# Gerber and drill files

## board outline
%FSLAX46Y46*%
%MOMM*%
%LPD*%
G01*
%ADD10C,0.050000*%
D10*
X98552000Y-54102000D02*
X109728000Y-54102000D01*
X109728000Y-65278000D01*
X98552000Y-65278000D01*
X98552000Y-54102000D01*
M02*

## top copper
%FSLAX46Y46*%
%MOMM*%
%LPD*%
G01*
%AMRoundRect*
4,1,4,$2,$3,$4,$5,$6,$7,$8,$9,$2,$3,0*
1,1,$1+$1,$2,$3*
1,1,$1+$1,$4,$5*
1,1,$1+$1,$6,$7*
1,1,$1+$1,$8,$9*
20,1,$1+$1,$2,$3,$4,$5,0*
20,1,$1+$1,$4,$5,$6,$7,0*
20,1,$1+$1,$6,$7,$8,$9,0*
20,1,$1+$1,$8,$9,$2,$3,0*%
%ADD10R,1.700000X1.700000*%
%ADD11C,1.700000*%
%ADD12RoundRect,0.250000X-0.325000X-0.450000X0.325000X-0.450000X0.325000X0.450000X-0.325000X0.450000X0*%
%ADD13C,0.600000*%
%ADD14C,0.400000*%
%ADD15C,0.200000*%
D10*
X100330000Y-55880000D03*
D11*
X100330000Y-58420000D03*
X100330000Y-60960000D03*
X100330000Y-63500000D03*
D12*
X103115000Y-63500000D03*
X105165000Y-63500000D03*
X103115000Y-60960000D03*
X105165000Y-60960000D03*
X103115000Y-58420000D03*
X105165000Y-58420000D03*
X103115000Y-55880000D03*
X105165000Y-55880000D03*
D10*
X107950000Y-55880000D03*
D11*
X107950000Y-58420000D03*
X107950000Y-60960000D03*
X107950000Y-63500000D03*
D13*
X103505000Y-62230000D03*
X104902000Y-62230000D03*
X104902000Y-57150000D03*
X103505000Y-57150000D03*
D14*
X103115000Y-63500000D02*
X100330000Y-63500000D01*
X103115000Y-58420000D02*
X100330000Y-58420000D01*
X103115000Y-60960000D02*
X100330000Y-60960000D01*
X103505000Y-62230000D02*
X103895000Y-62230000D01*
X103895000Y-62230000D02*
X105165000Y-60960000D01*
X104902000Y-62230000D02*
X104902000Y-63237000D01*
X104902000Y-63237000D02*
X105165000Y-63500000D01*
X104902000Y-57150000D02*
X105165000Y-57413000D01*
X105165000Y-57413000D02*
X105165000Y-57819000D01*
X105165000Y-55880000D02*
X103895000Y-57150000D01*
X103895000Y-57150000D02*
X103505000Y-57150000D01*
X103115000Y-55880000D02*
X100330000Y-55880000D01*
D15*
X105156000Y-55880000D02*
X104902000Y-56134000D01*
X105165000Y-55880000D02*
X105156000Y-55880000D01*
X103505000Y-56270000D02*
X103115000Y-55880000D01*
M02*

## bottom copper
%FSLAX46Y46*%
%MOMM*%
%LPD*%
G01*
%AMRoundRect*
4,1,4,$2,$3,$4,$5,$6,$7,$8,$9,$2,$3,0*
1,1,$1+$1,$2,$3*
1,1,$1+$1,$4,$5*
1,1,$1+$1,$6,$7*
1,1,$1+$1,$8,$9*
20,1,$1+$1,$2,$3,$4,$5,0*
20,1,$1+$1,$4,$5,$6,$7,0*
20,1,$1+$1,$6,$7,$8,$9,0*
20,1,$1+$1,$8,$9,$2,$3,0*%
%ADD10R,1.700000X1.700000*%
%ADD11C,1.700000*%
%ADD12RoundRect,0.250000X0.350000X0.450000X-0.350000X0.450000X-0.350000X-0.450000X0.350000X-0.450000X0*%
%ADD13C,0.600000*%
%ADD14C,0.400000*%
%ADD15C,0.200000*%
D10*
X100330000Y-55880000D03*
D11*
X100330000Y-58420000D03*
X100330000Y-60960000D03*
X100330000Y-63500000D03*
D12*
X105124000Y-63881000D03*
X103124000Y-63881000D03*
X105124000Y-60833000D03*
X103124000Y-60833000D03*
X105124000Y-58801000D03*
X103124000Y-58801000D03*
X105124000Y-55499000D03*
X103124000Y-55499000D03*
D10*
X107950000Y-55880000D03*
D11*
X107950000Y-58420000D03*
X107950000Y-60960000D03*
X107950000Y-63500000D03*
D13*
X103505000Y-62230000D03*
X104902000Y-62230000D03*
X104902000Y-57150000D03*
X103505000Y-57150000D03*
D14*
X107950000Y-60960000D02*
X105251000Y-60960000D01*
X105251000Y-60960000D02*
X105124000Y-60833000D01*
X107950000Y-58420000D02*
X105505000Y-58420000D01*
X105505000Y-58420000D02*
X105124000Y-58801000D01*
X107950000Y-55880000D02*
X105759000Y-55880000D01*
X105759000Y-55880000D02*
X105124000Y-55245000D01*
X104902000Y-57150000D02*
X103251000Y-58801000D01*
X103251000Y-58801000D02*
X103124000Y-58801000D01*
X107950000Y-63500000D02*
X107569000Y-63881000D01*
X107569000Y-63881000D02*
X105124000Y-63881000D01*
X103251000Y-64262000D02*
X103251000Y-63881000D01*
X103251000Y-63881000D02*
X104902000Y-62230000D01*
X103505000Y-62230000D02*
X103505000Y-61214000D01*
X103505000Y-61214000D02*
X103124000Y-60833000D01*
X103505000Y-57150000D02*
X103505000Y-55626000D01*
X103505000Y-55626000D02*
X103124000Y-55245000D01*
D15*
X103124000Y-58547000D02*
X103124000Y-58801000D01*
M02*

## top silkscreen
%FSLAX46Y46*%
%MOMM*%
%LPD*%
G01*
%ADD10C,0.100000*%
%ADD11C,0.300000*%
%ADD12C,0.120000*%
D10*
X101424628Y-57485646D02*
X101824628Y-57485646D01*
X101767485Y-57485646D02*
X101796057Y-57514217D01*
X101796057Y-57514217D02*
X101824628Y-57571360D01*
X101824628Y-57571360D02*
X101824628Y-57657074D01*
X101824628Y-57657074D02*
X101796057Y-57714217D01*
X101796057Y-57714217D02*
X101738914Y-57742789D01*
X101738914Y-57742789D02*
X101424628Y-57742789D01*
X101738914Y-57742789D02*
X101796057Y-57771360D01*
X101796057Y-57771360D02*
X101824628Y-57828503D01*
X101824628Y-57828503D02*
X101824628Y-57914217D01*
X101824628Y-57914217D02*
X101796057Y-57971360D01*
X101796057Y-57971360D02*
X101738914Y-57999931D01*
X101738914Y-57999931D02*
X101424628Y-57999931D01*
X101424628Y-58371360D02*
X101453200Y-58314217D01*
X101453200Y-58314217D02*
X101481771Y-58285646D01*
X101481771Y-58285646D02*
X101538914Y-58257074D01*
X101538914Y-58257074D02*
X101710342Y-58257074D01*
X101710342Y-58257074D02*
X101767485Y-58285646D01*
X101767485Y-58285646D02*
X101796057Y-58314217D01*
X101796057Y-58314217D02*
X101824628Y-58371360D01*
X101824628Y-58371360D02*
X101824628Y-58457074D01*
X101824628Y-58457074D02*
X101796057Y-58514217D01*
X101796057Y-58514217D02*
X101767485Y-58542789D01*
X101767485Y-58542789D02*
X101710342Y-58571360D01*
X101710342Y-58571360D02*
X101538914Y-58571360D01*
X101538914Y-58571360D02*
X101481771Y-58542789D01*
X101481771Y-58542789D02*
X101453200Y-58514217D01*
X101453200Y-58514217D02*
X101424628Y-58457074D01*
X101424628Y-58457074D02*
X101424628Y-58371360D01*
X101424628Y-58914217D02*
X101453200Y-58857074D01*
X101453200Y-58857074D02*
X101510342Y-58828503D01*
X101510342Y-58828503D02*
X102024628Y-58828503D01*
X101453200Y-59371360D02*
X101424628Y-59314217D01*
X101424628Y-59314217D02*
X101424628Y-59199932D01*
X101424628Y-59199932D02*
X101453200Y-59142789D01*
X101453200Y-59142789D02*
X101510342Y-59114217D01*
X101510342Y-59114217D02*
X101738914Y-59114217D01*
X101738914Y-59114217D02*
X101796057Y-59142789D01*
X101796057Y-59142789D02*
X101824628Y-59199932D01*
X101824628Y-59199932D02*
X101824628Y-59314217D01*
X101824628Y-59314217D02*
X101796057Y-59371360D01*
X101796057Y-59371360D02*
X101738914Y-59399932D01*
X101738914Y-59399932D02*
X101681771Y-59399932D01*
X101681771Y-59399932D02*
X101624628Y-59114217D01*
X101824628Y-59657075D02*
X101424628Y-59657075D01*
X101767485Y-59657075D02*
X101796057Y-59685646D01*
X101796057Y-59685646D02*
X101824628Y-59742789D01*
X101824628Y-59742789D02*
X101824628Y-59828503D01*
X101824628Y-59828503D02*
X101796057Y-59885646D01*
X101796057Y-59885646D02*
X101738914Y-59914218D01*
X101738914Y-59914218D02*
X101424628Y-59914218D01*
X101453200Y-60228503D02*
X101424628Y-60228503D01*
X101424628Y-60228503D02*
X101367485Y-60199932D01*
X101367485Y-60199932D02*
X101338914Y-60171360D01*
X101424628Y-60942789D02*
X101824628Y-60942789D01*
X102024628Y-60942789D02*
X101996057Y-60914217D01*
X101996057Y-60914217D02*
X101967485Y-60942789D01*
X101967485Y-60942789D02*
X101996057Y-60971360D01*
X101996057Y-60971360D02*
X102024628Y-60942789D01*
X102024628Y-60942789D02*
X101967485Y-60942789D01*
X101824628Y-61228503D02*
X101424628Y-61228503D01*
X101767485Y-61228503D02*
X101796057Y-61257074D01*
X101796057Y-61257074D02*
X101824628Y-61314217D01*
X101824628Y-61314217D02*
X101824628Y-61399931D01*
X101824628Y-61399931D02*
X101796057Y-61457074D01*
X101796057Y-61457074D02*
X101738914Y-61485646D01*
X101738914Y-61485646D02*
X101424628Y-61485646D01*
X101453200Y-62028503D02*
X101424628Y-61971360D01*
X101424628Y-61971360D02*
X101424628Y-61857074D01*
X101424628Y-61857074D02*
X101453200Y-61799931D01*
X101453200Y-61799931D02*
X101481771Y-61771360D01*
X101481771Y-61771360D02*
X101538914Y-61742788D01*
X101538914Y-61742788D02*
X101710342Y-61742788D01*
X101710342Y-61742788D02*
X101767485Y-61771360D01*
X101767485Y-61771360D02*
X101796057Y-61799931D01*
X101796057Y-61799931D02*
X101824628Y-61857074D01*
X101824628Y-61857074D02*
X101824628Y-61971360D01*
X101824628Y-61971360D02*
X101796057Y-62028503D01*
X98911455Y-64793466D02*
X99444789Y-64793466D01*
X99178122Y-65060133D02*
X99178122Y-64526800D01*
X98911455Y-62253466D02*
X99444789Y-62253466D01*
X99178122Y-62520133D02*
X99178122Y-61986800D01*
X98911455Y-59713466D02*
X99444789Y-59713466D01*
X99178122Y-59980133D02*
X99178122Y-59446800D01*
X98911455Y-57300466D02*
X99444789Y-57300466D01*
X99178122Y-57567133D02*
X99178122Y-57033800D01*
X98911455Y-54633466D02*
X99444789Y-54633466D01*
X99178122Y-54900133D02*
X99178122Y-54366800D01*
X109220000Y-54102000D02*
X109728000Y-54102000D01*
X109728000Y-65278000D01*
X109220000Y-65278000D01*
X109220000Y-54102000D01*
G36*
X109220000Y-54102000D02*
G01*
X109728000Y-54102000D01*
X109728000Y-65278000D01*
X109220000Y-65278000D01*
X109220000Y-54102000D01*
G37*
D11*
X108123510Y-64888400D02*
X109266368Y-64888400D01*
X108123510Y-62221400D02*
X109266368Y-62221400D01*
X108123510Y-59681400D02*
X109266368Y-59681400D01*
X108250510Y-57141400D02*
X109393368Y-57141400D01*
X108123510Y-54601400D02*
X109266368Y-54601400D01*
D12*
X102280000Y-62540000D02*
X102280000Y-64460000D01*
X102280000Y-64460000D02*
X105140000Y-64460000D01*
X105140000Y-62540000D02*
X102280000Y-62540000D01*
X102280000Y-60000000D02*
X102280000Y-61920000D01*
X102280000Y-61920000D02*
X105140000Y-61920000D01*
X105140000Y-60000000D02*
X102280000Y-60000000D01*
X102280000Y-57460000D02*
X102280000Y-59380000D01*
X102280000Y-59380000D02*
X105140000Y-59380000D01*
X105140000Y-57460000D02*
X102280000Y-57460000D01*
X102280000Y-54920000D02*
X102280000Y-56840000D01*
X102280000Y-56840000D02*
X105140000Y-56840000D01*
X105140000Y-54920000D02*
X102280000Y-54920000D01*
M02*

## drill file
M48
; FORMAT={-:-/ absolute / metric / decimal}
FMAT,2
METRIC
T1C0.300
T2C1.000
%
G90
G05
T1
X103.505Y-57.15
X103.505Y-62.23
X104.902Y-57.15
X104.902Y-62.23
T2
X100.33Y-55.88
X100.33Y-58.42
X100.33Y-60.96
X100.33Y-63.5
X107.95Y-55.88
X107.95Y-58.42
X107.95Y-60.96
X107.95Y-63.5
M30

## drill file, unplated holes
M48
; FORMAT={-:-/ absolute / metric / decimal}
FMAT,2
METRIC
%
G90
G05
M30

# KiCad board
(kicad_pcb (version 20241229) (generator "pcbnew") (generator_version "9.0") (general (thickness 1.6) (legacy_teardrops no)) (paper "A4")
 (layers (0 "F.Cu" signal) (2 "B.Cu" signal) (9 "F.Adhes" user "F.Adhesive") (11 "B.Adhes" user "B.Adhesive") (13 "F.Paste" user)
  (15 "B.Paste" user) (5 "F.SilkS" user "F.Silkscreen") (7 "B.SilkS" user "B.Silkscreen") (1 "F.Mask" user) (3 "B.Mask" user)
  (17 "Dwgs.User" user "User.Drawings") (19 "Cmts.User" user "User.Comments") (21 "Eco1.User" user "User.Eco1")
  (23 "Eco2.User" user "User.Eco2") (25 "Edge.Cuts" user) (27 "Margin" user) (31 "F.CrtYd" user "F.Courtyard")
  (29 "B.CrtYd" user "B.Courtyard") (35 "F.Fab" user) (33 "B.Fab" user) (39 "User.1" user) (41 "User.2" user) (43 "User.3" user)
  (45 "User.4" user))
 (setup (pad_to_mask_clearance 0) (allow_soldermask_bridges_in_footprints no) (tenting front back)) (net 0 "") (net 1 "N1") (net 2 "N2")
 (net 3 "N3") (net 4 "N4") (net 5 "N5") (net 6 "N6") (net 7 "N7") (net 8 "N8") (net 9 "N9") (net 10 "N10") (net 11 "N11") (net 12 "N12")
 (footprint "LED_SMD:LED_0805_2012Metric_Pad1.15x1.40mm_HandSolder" (layer "F.Cu") (at 104.14 63.5)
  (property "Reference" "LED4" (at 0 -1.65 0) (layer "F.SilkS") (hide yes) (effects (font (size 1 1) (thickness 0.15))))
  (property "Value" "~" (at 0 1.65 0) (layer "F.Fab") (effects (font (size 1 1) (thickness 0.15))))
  (fp_line (start -1.86 -0.96) (end -1.86 0.96) (stroke (width 0.12) (type solid)) (layer "F.SilkS"))
  (fp_line (start -1.86 0.96) (end 1 0.96) (stroke (width 0.12) (type solid)) (layer "F.SilkS"))
  (fp_line (start 1 -0.96) (end -1.86 -0.96) (stroke (width 0.12) (type solid)) (layer "F.SilkS"))
  (pad "1" smd roundrect (at -1.025 0) (size 1.15 1.4) (layers "F.Cu" "F.Mask" "F.Paste") (roundrect_rratio 0.217391) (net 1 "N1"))
  (pad "2" smd roundrect (at 1.025 0) (size 1.15 1.4) (layers "F.Cu" "F.Mask" "F.Paste") (roundrect_rratio 0.217391) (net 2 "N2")))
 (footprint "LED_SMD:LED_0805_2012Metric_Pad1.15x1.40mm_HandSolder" (layer "F.Cu") (at 104.14 60.96)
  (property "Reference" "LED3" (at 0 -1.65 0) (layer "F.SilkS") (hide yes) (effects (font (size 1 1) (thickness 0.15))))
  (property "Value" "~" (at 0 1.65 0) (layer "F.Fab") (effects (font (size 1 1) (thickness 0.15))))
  (fp_line (start -1.86 -0.96) (end -1.86 0.96) (stroke (width 0.12) (type solid)) (layer "F.SilkS"))
  (fp_line (start -1.86 0.96) (end 1 0.96) (stroke (width 0.12) (type solid)) (layer "F.SilkS"))
  (fp_line (start 1 -0.96) (end -1.86 -0.96) (stroke (width 0.12) (type solid)) (layer "F.SilkS"))
  (pad "1" smd roundrect (at -1.025 0) (size 1.15 1.4) (layers "F.Cu" "F.Mask" "F.Paste") (roundrect_rratio 0.217391) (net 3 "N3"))
  (pad "2" smd roundrect (at 1.025 0) (size 1.15 1.4) (layers "F.Cu" "F.Mask" "F.Paste") (roundrect_rratio 0.217391) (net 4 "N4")))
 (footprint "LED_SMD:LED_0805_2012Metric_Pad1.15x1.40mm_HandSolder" (layer "F.Cu") (at 104.14 55.88)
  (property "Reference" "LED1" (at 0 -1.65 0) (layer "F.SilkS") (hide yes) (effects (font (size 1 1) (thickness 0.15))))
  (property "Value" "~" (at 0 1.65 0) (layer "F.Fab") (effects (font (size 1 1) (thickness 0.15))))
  (fp_line (start -1.86 -0.96) (end -1.86 0.96) (stroke (width 0.12) (type solid)) (layer "F.SilkS"))
  (fp_line (start -1.86 0.96) (end 1 0.96) (stroke (width 0.12) (type solid)) (layer "F.SilkS"))
  (fp_line (start 1 -0.96) (end -1.86 -0.96) (stroke (width 0.12) (type solid)) (layer "F.SilkS"))
  (pad "1" smd roundrect (at -1.025 0) (size 1.15 1.4) (layers "F.Cu" "F.Mask" "F.Paste") (roundrect_rratio 0.217391) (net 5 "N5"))
  (pad "2" smd roundrect (at 1.025 0) (size 1.15 1.4) (layers "F.Cu" "F.Mask" "F.Paste") (roundrect_rratio 0.217391) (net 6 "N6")))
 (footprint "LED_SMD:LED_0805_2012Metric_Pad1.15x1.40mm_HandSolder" (layer "F.Cu") (at 104.14 58.42)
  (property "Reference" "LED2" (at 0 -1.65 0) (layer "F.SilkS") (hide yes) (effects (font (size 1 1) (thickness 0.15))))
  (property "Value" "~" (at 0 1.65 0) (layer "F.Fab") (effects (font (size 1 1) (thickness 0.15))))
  (fp_line (start -1.86 -0.96) (end -1.86 0.96) (stroke (width 0.12) (type solid)) (layer "F.SilkS"))
  (fp_line (start -1.86 0.96) (end 1 0.96) (stroke (width 0.12) (type solid)) (layer "F.SilkS"))
  (fp_line (start 1 -0.96) (end -1.86 -0.96) (stroke (width 0.12) (type solid)) (layer "F.SilkS"))
  (pad "1" smd roundrect (at -1.025 0) (size 1.15 1.4) (layers "F.Cu" "F.Mask" "F.Paste") (roundrect_rratio 0.217391) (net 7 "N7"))
  (pad "2" smd roundrect (at 1.025 0) (size 1.15 1.4) (layers "F.Cu" "F.Mask" "F.Paste") (roundrect_rratio 0.217391) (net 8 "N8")))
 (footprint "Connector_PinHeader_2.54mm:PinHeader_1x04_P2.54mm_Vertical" (layer "B.Cu") (at 100.33 55.88 180)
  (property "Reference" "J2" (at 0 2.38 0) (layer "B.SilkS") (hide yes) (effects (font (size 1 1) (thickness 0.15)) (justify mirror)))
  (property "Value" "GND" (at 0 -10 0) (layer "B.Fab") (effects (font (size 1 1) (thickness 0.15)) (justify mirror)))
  (pad "1" thru_hole rect (at 0 0 180) (size 1.7 1.7) (drill 1) (layers "*.Cu" "*.Mask") (remove_unused_layers no) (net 5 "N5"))
  (pad "2" thru_hole circle (at 0 -2.54 180) (size 1.7 1.7) (drill 1) (layers "*.Cu" "*.Mask") (remove_unused_layers no) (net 7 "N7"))
  (pad "3" thru_hole circle (at 0 -5.08 180) (size 1.7 1.7) (drill 1) (layers "*.Cu" "*.Mask") (remove_unused_layers no) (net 3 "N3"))
  (pad "4" thru_hole circle (at 0 -7.62 180) (size 1.7 1.7) (drill 1) (layers "*.Cu" "*.Mask") (remove_unused_layers no) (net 1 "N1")))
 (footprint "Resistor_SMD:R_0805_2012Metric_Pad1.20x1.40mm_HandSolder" (layer "B.Cu") (at 104.124 55.499 180)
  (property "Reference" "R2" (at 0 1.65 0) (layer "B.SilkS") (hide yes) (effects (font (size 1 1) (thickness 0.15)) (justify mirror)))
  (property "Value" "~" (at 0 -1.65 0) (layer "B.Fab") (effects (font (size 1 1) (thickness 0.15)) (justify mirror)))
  (pad "1" smd roundrect (at -1 0 180) (size 1.2 1.4) (layers "B.Cu" "B.Mask" "B.Paste") (roundrect_rratio 0.208333) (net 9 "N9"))
  (pad "2" smd roundrect (at 1 0 180) (size 1.2 1.4) (layers "B.Cu" "B.Mask" "B.Paste") (roundrect_rratio 0.208333) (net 6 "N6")))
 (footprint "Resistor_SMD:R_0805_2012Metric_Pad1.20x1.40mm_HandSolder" (layer "B.Cu") (at 104.124 60.833 180)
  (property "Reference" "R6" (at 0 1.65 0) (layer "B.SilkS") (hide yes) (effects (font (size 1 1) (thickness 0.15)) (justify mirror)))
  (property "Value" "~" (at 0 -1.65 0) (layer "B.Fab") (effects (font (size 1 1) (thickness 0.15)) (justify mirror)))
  (pad "1" smd roundrect (at -1 0 180) (size 1.2 1.4) (layers "B.Cu" "B.Mask" "B.Paste") (roundrect_rratio 0.208333) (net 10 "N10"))
  (pad "2" smd roundrect (at 1 0 180) (size 1.2 1.4) (layers "B.Cu" "B.Mask" "B.Paste") (roundrect_rratio 0.208333) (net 4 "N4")))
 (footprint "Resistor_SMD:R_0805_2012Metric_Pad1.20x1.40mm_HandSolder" (layer "B.Cu") (at 104.124 58.801 180)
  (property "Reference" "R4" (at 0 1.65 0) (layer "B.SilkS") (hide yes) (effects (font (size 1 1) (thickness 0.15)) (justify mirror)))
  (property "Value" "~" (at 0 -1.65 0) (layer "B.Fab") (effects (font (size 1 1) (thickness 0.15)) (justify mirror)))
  (pad "1" smd roundrect (at -1 0 180) (size 1.2 1.4) (layers "B.Cu" "B.Mask" "B.Paste") (roundrect_rratio 0.208333) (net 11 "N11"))
  (pad "2" smd roundrect (at 1 0 180) (size 1.2 1.4) (layers "B.Cu" "B.Mask" "B.Paste") (roundrect_rratio 0.208333) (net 8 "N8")))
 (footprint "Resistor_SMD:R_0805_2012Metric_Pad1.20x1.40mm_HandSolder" (layer "B.Cu") (at 104.124 63.881 180)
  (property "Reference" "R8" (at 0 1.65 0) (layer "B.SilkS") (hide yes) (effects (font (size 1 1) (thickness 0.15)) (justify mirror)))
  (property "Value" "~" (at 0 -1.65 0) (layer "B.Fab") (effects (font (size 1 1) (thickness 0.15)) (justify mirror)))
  (pad "1" smd roundrect (at -1 0 180) (size 1.2 1.4) (layers "B.Cu" "B.Mask" "B.Paste") (roundrect_rratio 0.208333) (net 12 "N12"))
  (pad "2" smd roundrect (at 1 0 180) (size 1.2 1.4) (layers "B.Cu" "B.Mask" "B.Paste") (roundrect_rratio 0.208333) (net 2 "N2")))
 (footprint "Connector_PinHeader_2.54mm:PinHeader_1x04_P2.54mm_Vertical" (layer "B.Cu") (at 107.95 55.88 180)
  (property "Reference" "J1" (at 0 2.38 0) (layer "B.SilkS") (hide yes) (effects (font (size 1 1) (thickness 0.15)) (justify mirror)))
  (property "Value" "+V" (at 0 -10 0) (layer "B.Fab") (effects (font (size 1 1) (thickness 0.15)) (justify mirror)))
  (pad "1" thru_hole rect (at 0 0 180) (size 1.7 1.7) (drill 1) (layers "*.Cu" "*.Mask") (remove_unused_layers no) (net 9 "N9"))
  (pad "2" thru_hole circle (at 0 -2.54 180) (size 1.7 1.7) (drill 1) (layers "*.Cu" "*.Mask") (remove_unused_layers no) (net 11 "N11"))
  (pad "3" thru_hole circle (at 0 -5.08 180) (size 1.7 1.7) (drill 1) (layers "*.Cu" "*.Mask") (remove_unused_layers no) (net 10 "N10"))
  (pad "4" thru_hole circle (at 0 -7.62 180) (size 1.7 1.7) (drill 1) (layers "*.Cu" "*.Mask") (remove_unused_layers no) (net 12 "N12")))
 (gr_rect (start 109.22 54.102) (end 109.728 65.278) (stroke (width 0.1) (type default)) (fill yes) (layer "F.SilkS"))
 (gr_rect (start 98.552 54.102) (end 109.728 65.278) (stroke (width 0.05) (type default)) (fill no) (layer "Edge.Cuts"))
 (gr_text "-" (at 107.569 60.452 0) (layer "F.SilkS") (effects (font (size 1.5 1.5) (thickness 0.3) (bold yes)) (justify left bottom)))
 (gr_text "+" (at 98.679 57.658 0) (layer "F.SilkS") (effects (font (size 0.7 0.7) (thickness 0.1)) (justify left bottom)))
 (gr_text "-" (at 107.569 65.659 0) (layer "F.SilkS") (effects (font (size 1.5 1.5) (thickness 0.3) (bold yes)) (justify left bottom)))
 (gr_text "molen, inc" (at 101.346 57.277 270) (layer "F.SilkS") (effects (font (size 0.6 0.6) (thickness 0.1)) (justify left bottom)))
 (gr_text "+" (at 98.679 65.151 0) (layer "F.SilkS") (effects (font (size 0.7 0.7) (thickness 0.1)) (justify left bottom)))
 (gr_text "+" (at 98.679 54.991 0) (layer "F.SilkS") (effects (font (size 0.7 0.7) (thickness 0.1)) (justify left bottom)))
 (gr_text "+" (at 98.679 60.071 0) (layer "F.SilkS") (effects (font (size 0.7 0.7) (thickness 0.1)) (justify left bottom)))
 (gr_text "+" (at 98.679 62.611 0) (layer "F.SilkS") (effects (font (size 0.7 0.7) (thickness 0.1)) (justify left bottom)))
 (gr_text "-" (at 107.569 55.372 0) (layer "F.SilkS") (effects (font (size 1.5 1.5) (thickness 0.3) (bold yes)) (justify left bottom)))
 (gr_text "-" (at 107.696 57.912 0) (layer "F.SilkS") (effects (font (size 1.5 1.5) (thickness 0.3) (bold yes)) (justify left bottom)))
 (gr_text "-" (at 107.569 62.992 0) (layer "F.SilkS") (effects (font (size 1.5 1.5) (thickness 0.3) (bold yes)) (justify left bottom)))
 (segment (start 105.251 60.96) (end 105.124 60.833) (width 0.4) (layer "B.Cu") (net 10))
 (segment (start 107.95 60.96) (end 105.251 60.96) (width 0.4) (layer "B.Cu") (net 10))
 (segment (start 107.569 63.881) (end 105.124 63.881) (width 0.4) (layer "B.Cu") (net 12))
 (segment (start 107.95 63.5) (end 107.569 63.881) (width 0.4) (layer "B.Cu") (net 12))
 (segment (start 107.95 58.42) (end 105.505 58.42) (width 0.4) (layer "B.Cu") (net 11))
 (segment (start 105.505 58.42) (end 105.124 58.801) (width 0.4) (layer "B.Cu") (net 11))
 (segment (start 107.95 55.88) (end 105.759 55.88) (width 0.4) (layer "B.Cu") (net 9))
 (segment (start 105.759 55.88) (end 105.124 55.245) (width 0.4) (layer "B.Cu") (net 9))
 (segment (start 103.115 58.42) (end 100.33 58.42) (width 0.4) (layer "F.Cu") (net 7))
 (segment (start 103.115 60.96) (end 100.33 60.96) (width 0.4) (layer "F.Cu") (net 3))
 (segment (start 103.115 63.5) (end 100.33 63.5) (width 0.4) (layer "F.Cu") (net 1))
 (segment (start 103.115 55.88) (end 100.33 55.88) (width 0.4) (layer "F.Cu") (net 5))
 (segment (start 103.505 56.27) (end 103.115 55.88) (width 0.2) (layer "F.Cu") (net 5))
 (segment (start 103.895 57.15) (end 103.505 57.15) (width 0.4) (layer "F.Cu") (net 6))
 (segment (start 105.156 55.88) (end 104.902 56.134) (width 0.2) (layer "F.Cu") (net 6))
 (segment (start 105.165 55.88) (end 103.895 57.15) (width 0.4) (layer "F.Cu") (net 6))
 (segment (start 105.165 55.88) (end 105.156 55.88) (width 0.2) (layer "F.Cu") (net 6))
 (via (at 103.505 57.15) (size 0.6) (drill 0.3) (layers "F.Cu" "B.Cu") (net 6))
 (segment (start 103.505 55.626) (end 103.124 55.245) (width 0.4) (layer "B.Cu") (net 6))
 (segment (start 103.505 57.15) (end 103.505 55.626) (width 0.4) (layer "B.Cu") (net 6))
 (segment (start 104.902 57.15) (end 105.165 57.413) (width 0.4) (layer "F.Cu") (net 8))
 (segment (start 105.165 57.413) (end 105.165 57.819) (width 0.4) (layer "F.Cu") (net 8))
 (via (at 104.902 57.15) (size 0.6) (drill 0.3) (layers "F.Cu" "B.Cu") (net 8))
 (segment (start 103.251 58.801) (end 103.124 58.801) (width 0.4) (layer "B.Cu") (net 8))
 (segment (start 103.124 58.547) (end 103.124 58.801) (width 0.2) (layer "B.Cu") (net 8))
 (segment (start 104.902 57.15) (end 103.251 58.801) (width 0.4) (layer "B.Cu") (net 8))
 (segment (start 103.895 62.23) (end 105.165 60.96) (width 0.4) (layer "F.Cu") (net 4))
 (segment (start 103.505 62.23) (end 103.895 62.23) (width 0.4) (layer "F.Cu") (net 4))
 (via (at 103.505 62.23) (size 0.6) (drill 0.3) (layers "F.Cu" "B.Cu") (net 4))
 (segment (start 103.505 61.214) (end 103.124 60.833) (width 0.4) (layer "B.Cu") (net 4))
 (segment (start 103.505 62.23) (end 103.505 61.214) (width 0.4) (layer "B.Cu") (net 4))
 (segment (start 104.902 62.23) (end 104.902 63.237) (width 0.4) (layer "F.Cu") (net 2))
 (segment (start 104.902 63.237) (end 105.165 63.5) (width 0.4) (layer "F.Cu") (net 2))
 (via (at 104.902 62.23) (size 0.6) (drill 0.3) (layers "F.Cu" "B.Cu") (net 2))
 (segment (start 103.251 64.262) (end 103.251 63.881) (width 0.4) (layer "B.Cu") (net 2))
 (segment (start 103.251 63.881) (end 104.902 62.23) (width 0.4) (layer "B.Cu") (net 2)))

